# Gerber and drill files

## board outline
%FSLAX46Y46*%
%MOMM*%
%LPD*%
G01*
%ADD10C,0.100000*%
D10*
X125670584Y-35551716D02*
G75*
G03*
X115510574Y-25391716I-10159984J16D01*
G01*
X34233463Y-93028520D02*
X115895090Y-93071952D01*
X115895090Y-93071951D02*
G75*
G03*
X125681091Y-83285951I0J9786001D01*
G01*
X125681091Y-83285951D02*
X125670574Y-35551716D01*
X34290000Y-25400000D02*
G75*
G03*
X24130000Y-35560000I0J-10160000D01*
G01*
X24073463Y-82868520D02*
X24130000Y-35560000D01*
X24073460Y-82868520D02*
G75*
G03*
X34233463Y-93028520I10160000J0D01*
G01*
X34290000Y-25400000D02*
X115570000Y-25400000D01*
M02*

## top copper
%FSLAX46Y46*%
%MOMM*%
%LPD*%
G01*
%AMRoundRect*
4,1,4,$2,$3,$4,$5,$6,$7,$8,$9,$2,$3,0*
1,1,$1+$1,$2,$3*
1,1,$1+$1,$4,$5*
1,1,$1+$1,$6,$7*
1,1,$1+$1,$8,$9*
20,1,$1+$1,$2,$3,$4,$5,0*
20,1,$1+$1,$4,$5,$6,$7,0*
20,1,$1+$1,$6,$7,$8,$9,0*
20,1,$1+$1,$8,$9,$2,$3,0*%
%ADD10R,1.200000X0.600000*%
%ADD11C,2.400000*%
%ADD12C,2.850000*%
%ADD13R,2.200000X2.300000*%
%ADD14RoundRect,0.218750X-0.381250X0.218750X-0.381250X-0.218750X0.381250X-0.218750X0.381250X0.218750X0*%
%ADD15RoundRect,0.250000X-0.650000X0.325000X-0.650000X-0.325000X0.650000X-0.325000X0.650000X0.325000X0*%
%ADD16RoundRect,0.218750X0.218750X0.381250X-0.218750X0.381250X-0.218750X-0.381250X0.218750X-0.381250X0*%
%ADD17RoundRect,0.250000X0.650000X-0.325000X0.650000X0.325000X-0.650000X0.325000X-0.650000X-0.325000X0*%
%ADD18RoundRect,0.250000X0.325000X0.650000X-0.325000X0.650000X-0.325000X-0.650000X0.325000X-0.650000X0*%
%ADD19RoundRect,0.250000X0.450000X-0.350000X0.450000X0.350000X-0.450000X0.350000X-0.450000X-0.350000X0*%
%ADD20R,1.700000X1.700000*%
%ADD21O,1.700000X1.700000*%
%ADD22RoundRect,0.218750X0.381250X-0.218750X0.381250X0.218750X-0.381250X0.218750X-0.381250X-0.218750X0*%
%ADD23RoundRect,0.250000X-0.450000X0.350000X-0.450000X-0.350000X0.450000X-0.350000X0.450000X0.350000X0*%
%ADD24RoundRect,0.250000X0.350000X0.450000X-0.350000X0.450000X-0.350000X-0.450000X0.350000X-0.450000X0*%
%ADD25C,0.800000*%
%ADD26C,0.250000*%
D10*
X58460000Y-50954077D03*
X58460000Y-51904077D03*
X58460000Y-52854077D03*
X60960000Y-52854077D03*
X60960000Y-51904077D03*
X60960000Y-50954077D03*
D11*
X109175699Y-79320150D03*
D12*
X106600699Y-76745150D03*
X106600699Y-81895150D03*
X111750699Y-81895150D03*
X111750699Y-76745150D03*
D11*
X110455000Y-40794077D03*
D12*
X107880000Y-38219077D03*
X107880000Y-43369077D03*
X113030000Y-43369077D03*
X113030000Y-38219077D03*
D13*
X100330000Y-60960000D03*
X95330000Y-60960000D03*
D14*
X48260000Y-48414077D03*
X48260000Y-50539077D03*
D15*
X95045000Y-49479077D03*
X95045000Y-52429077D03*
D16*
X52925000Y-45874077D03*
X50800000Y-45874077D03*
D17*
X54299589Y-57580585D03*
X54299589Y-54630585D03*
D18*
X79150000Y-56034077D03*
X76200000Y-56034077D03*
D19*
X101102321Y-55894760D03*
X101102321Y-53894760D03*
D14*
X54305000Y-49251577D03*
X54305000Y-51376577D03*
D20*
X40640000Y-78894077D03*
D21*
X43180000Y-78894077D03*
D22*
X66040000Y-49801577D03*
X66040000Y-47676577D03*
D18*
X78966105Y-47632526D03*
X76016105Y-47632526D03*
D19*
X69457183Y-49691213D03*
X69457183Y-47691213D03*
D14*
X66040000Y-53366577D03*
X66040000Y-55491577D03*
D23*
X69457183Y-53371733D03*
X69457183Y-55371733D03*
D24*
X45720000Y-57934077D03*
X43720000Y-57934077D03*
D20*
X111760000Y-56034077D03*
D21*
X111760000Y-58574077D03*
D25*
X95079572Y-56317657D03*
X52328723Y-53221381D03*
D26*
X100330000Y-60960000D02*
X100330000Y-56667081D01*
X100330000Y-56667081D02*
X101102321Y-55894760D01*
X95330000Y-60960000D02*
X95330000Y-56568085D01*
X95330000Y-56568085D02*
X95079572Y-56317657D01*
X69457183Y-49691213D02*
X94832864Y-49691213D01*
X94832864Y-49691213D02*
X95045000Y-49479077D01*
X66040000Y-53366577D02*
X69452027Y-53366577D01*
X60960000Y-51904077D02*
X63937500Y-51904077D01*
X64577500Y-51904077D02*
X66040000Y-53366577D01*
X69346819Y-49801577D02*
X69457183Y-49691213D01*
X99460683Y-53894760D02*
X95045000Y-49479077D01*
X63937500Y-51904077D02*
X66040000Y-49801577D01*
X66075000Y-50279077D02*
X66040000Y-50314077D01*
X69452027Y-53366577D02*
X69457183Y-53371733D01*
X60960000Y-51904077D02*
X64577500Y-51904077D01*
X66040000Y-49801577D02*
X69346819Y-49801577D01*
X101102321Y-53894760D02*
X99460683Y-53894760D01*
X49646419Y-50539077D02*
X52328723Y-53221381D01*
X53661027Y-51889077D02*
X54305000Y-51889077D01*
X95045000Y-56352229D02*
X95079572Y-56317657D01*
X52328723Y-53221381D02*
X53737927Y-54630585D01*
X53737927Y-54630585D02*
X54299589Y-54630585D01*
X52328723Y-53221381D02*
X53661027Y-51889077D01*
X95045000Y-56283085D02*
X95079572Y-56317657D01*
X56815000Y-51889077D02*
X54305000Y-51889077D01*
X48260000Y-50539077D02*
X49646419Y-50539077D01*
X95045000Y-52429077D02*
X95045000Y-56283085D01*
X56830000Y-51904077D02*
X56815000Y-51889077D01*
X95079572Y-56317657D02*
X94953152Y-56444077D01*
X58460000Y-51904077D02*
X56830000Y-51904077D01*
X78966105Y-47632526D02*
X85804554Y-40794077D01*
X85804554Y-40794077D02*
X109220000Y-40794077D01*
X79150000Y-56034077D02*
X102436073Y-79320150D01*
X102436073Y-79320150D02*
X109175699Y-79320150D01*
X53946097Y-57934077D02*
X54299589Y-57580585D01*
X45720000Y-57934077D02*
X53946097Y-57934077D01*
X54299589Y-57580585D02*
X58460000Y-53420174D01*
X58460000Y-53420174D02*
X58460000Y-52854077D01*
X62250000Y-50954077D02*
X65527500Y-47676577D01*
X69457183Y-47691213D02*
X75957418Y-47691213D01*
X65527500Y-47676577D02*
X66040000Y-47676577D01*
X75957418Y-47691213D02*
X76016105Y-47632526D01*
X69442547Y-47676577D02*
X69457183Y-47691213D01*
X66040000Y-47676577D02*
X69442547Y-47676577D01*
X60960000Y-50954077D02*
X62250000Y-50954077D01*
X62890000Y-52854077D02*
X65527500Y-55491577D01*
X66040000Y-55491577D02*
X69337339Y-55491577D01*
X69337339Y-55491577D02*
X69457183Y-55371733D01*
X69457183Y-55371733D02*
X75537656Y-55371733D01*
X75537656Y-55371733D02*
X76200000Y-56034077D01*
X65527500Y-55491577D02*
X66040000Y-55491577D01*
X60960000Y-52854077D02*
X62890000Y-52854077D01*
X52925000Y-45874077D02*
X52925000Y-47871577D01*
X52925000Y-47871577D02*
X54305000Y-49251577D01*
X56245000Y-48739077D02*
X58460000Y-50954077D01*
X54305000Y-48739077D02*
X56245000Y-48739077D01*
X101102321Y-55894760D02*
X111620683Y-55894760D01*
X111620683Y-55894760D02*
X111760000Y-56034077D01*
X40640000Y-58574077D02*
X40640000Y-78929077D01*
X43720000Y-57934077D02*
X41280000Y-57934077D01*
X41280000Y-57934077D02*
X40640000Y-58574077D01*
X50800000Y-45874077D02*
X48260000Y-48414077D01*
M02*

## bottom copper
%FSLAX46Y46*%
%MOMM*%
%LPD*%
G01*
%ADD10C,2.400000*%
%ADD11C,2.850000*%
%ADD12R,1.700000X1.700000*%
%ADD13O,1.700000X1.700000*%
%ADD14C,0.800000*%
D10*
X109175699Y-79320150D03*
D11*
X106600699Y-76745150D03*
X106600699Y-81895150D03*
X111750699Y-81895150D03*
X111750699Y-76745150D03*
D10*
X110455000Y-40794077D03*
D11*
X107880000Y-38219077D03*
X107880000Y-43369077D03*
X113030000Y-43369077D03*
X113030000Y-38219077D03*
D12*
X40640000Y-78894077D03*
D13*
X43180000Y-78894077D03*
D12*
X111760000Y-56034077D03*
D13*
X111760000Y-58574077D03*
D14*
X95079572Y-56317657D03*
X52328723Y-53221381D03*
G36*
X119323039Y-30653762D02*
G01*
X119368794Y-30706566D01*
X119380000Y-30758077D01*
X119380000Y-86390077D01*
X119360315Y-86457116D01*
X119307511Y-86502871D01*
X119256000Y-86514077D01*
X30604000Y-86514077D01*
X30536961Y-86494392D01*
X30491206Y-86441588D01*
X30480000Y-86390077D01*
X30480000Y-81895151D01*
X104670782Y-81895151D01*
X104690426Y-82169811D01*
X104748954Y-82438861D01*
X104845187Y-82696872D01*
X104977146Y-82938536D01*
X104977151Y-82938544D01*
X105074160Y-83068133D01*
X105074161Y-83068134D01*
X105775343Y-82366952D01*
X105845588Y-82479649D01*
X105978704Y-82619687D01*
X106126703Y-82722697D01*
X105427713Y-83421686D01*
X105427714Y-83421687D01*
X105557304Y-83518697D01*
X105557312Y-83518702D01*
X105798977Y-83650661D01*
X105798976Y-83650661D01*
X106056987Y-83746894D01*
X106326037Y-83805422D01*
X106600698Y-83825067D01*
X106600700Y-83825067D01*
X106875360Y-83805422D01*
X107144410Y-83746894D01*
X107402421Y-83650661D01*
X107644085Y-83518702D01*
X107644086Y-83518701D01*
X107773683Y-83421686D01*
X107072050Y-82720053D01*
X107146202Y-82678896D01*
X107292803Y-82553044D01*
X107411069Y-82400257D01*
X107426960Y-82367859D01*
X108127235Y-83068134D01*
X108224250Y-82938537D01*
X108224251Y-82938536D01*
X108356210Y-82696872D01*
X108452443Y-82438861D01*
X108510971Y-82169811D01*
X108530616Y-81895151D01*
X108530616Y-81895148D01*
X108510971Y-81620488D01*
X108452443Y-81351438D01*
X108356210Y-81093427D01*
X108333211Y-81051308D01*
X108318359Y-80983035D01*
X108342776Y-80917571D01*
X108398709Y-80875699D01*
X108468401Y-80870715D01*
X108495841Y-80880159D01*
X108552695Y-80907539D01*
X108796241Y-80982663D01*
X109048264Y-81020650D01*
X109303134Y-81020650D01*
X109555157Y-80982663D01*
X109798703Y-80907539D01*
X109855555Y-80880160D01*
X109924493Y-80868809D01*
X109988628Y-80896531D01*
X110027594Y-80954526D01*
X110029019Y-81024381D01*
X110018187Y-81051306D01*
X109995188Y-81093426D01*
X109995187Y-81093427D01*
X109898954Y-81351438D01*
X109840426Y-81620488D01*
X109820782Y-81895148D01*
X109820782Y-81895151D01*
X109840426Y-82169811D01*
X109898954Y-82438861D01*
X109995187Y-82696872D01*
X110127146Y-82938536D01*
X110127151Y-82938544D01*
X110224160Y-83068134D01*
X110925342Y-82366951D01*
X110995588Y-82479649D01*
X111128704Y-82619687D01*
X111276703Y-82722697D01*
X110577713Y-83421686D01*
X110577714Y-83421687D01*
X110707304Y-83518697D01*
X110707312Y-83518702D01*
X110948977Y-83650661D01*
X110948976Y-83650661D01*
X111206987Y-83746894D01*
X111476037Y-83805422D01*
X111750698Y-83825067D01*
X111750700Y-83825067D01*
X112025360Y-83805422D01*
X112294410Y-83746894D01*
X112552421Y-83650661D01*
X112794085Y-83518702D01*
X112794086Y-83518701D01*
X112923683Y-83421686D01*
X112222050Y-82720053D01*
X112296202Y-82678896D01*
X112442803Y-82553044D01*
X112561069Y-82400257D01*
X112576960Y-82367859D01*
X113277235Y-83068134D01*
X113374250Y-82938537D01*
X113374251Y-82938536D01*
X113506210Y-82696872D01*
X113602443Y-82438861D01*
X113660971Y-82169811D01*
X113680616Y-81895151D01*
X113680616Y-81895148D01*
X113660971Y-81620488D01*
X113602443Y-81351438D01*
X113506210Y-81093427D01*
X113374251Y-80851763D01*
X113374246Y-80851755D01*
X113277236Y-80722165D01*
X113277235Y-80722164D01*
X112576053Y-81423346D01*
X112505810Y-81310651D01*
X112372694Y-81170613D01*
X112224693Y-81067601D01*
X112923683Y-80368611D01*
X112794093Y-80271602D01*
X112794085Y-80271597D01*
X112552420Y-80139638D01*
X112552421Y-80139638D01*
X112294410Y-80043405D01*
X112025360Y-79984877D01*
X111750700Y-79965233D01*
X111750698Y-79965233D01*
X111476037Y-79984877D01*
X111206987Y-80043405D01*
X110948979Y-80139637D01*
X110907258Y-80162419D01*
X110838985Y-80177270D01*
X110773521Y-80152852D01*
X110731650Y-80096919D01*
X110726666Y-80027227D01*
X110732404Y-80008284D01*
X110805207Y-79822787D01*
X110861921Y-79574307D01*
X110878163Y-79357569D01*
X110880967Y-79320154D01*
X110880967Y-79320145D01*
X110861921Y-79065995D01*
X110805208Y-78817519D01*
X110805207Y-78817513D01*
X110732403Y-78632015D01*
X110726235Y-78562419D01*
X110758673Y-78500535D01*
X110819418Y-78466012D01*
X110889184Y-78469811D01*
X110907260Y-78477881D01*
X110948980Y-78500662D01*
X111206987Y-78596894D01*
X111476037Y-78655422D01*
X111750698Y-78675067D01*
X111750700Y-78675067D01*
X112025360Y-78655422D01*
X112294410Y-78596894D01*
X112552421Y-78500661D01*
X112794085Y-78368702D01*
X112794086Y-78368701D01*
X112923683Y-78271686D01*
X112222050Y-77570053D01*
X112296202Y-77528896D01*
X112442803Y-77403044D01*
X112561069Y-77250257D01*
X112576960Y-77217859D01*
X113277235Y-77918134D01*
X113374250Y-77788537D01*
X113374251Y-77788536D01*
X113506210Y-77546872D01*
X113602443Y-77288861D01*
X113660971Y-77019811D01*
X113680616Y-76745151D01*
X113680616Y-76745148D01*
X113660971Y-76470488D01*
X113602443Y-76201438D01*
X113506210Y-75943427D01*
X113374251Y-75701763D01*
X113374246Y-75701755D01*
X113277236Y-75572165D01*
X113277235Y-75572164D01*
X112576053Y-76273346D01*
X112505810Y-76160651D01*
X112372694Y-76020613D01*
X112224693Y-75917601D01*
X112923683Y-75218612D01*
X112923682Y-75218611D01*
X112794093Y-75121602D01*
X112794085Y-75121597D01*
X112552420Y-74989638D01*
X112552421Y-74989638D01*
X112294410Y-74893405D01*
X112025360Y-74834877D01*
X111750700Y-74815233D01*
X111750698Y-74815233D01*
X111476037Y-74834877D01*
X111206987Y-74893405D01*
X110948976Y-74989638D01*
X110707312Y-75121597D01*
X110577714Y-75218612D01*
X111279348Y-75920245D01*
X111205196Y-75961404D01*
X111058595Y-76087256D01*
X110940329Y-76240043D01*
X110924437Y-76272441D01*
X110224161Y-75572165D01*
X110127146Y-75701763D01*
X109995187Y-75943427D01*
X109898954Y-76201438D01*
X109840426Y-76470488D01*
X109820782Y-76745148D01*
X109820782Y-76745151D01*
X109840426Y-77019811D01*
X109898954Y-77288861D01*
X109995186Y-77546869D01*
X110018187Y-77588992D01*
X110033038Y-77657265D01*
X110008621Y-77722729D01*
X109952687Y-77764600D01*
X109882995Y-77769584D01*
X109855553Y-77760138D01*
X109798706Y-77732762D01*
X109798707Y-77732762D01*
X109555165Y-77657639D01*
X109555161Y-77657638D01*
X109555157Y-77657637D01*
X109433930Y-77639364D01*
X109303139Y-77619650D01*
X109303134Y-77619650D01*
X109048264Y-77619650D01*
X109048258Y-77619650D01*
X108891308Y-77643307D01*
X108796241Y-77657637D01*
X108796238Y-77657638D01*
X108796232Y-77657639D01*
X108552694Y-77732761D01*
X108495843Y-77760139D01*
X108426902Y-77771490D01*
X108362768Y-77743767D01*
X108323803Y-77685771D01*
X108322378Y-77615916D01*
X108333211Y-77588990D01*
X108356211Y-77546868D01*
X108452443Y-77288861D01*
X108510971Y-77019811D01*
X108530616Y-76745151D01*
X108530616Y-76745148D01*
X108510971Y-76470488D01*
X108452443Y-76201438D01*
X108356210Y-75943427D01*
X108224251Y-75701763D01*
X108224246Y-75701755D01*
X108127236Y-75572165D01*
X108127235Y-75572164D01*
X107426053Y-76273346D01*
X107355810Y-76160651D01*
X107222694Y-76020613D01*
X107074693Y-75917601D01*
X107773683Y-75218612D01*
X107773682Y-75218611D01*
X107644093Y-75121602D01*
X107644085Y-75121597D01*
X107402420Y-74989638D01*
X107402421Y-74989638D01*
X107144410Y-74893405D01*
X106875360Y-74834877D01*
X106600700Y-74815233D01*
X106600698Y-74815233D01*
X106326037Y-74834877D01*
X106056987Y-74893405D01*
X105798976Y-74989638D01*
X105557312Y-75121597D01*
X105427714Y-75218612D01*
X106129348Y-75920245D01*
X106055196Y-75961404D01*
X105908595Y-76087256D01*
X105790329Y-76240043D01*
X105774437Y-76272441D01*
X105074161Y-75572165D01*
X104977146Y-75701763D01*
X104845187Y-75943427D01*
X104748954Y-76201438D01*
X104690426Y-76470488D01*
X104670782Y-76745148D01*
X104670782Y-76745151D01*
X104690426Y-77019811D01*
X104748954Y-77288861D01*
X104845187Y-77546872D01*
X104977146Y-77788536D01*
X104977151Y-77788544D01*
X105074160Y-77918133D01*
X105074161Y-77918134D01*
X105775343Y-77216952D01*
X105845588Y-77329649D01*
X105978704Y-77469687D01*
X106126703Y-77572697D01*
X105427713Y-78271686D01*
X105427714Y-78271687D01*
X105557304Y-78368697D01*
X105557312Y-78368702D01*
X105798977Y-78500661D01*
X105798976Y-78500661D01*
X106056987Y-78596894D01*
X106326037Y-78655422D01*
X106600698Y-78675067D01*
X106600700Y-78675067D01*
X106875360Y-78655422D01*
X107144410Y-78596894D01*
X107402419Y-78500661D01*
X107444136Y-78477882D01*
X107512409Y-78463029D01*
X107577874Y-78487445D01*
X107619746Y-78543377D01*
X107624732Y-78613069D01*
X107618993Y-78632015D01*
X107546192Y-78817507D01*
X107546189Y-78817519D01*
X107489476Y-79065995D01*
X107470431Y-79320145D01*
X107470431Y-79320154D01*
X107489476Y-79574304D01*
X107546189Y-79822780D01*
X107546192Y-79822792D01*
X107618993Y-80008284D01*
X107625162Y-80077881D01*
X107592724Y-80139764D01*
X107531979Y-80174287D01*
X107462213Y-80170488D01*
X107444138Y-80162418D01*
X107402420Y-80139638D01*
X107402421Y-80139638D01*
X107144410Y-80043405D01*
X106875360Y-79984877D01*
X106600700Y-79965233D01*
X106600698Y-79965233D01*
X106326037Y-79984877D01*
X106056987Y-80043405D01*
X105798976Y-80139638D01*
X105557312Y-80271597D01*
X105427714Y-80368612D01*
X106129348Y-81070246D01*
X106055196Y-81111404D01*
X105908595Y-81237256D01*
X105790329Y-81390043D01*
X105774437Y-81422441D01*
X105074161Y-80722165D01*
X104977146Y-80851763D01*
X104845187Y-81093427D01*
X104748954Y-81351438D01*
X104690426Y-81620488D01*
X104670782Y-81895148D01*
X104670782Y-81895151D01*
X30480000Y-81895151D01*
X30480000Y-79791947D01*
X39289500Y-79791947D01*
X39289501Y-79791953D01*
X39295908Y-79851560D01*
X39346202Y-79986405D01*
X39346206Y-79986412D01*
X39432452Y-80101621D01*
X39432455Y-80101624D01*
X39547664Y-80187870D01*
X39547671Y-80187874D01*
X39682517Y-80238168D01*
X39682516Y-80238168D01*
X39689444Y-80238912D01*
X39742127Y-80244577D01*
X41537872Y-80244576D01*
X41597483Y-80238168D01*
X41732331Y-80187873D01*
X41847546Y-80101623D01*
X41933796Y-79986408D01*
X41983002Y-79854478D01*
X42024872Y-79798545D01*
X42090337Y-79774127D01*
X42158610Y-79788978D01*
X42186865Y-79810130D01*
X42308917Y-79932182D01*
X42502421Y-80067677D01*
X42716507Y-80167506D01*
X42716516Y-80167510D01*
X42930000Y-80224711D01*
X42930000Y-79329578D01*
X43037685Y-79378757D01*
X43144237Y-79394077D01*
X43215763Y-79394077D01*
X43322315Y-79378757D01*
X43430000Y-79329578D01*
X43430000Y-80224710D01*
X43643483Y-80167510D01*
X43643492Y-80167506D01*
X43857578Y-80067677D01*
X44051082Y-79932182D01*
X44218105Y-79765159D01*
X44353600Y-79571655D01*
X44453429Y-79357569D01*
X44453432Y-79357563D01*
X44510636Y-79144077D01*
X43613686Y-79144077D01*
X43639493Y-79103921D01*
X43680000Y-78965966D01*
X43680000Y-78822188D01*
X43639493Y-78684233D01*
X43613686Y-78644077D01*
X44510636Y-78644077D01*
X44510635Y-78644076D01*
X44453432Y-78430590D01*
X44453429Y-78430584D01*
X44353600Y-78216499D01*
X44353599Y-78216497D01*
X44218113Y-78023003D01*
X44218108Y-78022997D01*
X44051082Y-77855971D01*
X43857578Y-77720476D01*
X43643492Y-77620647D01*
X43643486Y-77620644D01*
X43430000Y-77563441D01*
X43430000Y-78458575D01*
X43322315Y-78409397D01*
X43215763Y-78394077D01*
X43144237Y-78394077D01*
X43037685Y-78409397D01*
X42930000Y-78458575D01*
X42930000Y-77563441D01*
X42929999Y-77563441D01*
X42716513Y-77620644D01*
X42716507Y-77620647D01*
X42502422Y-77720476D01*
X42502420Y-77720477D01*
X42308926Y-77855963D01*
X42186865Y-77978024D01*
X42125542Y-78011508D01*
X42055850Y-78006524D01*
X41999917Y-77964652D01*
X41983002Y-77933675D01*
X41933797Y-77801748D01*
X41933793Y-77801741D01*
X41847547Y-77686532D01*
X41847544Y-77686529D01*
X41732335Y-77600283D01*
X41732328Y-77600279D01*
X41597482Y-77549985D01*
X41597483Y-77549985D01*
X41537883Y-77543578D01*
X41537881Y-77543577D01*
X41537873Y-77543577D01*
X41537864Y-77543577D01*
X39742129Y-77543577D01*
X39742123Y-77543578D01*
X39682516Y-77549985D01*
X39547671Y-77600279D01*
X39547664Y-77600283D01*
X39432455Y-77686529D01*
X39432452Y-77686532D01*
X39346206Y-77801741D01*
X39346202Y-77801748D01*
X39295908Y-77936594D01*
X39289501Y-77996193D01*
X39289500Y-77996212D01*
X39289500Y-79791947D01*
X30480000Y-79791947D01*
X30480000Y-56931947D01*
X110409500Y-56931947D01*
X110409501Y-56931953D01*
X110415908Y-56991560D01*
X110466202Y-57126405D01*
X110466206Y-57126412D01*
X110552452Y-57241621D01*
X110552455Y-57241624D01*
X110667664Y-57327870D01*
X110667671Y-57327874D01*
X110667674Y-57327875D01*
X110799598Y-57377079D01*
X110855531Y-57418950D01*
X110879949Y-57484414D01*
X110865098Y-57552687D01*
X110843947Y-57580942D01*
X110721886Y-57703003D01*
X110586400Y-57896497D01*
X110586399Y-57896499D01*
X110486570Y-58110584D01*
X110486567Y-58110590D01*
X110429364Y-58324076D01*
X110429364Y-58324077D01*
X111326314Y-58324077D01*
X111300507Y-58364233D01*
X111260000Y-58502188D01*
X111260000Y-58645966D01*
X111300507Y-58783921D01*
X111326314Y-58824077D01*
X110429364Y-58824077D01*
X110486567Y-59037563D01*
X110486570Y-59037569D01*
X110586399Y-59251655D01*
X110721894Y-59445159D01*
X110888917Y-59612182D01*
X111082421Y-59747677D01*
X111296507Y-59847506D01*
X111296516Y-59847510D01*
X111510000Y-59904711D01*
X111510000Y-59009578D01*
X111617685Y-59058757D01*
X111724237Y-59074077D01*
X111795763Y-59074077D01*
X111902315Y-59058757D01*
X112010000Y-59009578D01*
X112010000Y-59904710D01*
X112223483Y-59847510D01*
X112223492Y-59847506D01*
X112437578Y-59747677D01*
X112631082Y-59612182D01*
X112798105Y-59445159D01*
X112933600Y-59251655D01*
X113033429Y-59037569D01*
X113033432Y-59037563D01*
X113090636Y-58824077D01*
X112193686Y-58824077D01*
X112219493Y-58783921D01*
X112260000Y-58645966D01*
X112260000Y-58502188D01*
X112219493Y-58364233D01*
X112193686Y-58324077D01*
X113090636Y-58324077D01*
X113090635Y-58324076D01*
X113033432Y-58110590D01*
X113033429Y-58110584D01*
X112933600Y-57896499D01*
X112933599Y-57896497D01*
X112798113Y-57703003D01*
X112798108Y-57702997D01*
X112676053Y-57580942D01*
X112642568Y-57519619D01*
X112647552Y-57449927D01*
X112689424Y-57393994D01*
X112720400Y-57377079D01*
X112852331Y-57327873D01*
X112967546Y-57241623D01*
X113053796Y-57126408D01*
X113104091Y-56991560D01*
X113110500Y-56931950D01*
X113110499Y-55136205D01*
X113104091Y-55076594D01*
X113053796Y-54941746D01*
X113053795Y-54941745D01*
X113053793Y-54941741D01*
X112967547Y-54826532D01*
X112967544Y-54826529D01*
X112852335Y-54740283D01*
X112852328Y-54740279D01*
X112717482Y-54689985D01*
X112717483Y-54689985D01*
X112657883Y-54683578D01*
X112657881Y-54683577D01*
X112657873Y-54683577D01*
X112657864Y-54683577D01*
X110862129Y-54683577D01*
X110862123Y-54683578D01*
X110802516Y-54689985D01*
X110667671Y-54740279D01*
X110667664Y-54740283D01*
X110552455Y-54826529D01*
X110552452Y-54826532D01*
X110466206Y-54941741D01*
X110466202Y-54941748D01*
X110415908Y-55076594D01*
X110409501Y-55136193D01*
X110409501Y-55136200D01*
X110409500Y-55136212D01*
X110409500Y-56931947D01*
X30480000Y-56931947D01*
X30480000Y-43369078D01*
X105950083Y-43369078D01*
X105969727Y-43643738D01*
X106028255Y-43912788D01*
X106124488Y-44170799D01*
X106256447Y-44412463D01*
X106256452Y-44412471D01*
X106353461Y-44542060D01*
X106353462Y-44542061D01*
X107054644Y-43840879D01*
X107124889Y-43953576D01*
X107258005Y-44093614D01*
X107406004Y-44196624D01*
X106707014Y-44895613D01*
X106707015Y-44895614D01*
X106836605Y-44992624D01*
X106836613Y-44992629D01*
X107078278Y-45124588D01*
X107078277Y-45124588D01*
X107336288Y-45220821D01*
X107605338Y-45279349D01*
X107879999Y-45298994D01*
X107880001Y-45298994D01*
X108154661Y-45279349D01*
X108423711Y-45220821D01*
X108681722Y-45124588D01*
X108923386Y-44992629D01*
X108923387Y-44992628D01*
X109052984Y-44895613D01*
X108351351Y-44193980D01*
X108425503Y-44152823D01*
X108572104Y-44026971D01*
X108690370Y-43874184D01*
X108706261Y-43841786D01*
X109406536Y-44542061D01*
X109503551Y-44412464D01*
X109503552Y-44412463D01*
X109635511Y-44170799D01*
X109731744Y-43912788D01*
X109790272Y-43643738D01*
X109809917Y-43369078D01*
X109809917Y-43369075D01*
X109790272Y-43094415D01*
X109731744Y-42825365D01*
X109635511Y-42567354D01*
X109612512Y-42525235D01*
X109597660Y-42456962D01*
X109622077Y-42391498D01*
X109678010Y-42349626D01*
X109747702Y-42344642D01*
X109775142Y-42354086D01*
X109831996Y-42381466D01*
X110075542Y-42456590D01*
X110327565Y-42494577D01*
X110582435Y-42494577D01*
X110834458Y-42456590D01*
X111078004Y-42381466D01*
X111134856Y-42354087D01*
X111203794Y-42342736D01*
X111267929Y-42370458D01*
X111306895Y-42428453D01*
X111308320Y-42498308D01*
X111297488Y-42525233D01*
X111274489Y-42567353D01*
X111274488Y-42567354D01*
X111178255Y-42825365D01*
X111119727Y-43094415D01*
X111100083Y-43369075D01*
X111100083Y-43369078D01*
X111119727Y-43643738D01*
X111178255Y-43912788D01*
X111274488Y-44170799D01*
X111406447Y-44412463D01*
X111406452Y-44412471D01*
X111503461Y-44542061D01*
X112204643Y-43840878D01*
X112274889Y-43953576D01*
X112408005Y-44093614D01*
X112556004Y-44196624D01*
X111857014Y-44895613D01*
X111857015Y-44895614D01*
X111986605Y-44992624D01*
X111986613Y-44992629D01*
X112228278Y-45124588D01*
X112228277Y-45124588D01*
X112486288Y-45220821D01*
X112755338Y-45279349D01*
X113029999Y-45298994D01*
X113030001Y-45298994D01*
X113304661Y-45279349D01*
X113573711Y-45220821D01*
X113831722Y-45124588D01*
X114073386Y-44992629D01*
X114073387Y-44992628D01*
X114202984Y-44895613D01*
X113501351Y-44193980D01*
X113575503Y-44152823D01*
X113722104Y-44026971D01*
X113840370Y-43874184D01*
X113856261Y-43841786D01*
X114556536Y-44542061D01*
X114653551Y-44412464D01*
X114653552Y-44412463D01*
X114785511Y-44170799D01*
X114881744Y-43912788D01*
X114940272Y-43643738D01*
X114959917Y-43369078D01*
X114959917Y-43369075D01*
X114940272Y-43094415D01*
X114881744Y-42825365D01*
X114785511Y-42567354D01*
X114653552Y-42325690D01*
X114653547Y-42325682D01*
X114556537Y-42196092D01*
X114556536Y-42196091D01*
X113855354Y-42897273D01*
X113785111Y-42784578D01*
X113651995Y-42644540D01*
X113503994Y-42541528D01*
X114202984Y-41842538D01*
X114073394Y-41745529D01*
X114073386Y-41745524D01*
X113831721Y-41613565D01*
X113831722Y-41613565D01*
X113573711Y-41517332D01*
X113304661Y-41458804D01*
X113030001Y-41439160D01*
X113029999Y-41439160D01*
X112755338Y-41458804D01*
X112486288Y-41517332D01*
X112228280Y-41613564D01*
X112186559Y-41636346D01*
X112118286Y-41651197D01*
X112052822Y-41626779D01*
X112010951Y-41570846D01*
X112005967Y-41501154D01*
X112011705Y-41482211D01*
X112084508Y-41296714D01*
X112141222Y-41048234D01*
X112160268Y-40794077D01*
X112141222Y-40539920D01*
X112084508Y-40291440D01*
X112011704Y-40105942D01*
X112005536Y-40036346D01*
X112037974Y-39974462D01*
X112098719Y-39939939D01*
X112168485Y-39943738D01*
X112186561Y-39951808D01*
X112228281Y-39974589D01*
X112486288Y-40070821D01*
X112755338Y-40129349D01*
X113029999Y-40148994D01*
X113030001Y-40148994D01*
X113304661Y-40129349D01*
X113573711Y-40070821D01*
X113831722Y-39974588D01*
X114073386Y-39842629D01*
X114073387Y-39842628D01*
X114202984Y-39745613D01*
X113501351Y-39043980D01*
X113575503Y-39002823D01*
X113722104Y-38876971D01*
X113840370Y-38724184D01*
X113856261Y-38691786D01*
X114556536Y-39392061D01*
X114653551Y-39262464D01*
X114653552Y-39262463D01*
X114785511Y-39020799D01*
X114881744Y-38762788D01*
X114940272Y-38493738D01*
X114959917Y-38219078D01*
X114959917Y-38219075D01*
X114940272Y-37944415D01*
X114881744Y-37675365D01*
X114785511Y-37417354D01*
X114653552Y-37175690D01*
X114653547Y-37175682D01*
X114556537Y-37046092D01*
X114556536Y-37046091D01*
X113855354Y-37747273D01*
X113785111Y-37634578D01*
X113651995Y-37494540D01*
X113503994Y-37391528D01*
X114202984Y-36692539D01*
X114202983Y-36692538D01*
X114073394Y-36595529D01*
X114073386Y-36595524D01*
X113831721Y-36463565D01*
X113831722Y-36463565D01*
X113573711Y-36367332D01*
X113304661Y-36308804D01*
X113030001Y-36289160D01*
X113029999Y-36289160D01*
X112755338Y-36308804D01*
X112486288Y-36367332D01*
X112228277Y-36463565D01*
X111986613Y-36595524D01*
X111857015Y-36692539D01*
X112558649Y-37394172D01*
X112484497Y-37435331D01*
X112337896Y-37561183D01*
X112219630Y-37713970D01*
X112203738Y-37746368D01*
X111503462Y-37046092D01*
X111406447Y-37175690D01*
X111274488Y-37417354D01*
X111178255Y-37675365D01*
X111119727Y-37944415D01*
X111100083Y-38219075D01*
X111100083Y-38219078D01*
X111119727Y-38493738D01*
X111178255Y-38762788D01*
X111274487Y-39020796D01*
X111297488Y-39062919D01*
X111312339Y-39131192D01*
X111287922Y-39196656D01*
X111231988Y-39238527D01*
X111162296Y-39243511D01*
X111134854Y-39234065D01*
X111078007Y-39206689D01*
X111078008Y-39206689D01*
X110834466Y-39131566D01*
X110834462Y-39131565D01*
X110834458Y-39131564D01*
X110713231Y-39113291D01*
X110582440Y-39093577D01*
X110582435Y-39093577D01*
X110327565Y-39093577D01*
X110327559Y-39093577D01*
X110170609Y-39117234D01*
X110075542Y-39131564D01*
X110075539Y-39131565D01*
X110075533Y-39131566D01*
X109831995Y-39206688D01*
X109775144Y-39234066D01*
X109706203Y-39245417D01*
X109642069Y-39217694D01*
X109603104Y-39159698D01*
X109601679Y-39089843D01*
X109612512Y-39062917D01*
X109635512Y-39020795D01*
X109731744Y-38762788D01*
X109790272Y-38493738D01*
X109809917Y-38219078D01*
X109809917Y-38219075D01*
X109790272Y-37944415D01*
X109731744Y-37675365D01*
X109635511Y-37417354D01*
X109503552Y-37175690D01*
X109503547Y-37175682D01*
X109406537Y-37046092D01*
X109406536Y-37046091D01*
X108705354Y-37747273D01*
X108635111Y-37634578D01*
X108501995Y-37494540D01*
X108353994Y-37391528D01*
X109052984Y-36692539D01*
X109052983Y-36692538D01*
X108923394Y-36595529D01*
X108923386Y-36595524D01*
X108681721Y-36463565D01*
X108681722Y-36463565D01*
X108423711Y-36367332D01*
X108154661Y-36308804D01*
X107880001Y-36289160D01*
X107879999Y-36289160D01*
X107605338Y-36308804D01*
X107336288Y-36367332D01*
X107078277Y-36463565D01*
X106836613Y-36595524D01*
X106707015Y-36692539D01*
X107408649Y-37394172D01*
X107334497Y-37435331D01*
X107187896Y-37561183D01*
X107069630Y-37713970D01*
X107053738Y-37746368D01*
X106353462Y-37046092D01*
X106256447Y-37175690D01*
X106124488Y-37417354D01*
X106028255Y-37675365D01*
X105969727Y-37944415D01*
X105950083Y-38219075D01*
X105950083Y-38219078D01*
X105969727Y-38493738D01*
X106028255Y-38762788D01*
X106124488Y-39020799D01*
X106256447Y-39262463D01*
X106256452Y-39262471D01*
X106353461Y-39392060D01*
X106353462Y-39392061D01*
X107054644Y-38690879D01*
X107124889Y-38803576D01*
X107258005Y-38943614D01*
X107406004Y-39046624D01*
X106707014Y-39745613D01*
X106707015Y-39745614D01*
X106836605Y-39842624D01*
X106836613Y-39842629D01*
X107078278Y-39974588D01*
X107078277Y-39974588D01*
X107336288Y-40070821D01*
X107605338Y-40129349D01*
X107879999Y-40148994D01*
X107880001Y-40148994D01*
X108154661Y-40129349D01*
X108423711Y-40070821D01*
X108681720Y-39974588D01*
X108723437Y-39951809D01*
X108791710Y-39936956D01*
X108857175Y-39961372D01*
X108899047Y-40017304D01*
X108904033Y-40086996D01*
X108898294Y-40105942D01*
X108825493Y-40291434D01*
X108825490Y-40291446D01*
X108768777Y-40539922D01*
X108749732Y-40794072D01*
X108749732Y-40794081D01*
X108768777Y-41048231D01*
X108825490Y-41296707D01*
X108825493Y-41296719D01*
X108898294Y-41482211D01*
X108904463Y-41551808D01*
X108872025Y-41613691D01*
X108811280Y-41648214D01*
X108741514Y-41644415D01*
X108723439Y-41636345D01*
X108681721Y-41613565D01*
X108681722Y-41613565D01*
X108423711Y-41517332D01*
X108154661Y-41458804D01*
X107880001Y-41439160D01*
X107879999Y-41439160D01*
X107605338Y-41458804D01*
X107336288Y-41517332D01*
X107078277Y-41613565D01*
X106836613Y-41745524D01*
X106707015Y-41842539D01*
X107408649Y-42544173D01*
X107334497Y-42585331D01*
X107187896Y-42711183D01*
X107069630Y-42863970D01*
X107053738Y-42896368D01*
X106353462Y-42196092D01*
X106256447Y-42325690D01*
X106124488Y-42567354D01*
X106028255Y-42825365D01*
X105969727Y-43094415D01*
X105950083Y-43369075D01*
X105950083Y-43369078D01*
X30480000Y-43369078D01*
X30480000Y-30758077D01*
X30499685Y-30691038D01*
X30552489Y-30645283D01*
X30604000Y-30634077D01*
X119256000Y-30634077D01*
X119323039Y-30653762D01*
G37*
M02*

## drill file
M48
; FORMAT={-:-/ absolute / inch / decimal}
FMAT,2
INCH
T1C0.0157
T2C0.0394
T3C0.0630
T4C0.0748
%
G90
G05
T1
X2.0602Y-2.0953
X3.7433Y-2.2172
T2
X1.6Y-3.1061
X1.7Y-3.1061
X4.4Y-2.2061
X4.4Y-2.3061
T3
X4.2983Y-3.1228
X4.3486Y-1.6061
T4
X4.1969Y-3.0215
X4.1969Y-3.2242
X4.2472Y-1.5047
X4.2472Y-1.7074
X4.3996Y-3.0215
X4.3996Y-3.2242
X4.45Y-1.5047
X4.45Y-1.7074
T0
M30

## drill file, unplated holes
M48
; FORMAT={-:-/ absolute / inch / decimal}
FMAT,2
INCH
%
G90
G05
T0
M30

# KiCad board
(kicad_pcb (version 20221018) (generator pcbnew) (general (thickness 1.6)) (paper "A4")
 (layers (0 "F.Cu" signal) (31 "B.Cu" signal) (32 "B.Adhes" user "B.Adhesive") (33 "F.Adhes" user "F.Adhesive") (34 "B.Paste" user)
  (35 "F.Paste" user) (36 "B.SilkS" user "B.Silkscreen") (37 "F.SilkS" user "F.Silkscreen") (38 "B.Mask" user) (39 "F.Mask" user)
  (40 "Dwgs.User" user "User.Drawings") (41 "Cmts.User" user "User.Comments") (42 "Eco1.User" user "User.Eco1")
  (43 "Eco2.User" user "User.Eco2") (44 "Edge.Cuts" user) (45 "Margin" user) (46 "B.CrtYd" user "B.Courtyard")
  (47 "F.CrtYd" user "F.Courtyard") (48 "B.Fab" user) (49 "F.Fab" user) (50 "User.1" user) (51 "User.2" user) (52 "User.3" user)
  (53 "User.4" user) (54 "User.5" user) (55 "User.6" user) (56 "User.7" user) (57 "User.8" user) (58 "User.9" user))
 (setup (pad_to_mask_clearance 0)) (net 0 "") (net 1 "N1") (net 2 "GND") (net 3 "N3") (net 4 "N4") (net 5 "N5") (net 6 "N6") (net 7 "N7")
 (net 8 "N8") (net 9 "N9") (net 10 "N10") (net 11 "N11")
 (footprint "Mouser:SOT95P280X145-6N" (layer "F.Cu") (at 59.71 51.904077)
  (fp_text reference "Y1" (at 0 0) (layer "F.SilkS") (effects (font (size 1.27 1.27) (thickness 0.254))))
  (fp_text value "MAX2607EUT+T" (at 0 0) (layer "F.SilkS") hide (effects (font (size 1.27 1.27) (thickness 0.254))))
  (pad "1" smd rect (at -1.25 -0.95 90) (size 0.6 1.2) (layers "F.Cu" "F.Paste" "F.Mask") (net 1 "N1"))
  (pad "2" smd rect (at -1.25 0 90) (size 0.6 1.2) (layers "F.Cu" "F.Paste" "F.Mask") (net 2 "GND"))
  (pad "3" smd rect (at -1.25 0.95 90) (size 0.6 1.2) (layers "F.Cu" "F.Paste" "F.Mask") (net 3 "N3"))
  (pad "4" smd rect (at 1.25 0.95 90) (size 0.6 1.2) (layers "F.Cu" "F.Paste" "F.Mask") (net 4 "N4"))
  (pad "5" smd rect (at 1.25 0 90) (size 0.6 1.2) (layers "F.Cu" "F.Paste" "F.Mask") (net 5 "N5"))
  (pad "6" smd rect (at 1.25 -0.95 90) (size 0.6 1.2) (layers "F.Cu" "F.Paste" "F.Mask") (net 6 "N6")))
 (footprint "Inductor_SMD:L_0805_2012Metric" (layer "F.Cu") (at 48.26 49.476577 -90)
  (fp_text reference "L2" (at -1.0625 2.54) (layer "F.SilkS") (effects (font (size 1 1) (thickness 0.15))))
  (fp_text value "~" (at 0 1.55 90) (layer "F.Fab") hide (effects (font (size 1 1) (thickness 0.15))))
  (pad "1" smd roundrect (at -1.0625 0 270) (size 0.875 1.2) (layers "F.Cu" "F.Paste" "F.Mask") (roundrect_rratio 0.25) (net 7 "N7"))
  (pad "2" smd roundrect (at 1.0625 0 270) (size 0.875 1.2) (layers "F.Cu" "F.Paste" "F.Mask") (roundrect_rratio 0.25) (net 2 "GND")))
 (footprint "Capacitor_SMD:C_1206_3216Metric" (layer "F.Cu") (at 95.045 50.954077 -90)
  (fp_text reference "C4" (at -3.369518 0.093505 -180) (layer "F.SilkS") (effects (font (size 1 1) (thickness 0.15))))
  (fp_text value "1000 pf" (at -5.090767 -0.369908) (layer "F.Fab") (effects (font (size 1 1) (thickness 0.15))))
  (pad "1" smd roundrect (at -1.475 0 270) (size 1.15 1.8) (layers "F.Cu" "F.Paste" "F.Mask") (roundrect_rratio 0.2173913043) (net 5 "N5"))
  (pad "2" smd roundrect (at 1.475 0 270) (size 1.15 1.8) (layers "F.Cu" "F.Paste" "F.Mask") (roundrect_rratio 0.2173913043) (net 2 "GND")))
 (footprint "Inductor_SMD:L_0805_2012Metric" (layer "F.Cu") (at 51.8625 45.874077 180)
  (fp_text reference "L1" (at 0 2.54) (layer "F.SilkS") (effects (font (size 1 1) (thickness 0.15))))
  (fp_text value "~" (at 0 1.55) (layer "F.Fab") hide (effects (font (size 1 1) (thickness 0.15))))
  (pad "1" smd roundrect (at -1.0625 0 180) (size 0.875 1.2) (layers "F.Cu" "F.Paste" "F.Mask") (roundrect_rratio 0.25) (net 1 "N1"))
  (pad "2" smd roundrect (at 1.0625 0 180) (size 0.875 1.2) (layers "F.Cu" "F.Paste" "F.Mask") (roundrect_rratio 0.25) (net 7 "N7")))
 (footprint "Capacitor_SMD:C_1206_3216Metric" (layer "F.Cu") (at 54.299589 56.105585 90)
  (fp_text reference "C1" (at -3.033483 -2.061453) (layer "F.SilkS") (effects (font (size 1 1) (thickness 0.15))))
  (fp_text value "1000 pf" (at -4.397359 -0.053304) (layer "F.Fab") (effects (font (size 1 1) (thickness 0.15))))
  (pad "1" smd roundrect (at -1.475 0 90) (size 1.15 1.8) (layers "F.Cu" "F.Paste" "F.Mask") (roundrect_rratio 0.2173913043) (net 3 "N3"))
  (pad "2" smd roundrect (at 1.475 0 90) (size 1.15 1.8) (layers "F.Cu" "F.Paste" "F.Mask") (roundrect_rratio 0.2173913043) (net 2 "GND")))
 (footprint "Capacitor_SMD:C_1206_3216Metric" (layer "F.Cu") (at 77.675 56.034077 180)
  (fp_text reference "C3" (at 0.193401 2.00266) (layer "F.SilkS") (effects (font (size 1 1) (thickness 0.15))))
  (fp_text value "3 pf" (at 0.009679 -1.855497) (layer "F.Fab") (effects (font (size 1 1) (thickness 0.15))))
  (pad "1" smd roundrect (at -1.475 0 180) (size 1.15 1.8) (layers "F.Cu" "F.Paste" "F.Mask") (roundrect_rratio 0.2173913043) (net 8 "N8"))
  (pad "2" smd roundrect (at 1.475 0 180) (size 1.15 1.8) (layers "F.Cu" "F.Paste" "F.Mask") (roundrect_rratio 0.2173913043) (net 4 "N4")))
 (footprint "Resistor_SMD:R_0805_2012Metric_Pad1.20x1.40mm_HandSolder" (layer "F.Cu") (at 101.102321 54.89476 90)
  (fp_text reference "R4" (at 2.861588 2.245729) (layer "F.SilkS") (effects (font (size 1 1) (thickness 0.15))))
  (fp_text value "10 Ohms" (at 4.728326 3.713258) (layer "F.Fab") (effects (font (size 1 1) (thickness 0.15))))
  (pad "1" smd roundrect (at -1 0 90) (size 1.2 1.4) (layers "F.Cu" "F.Paste" "F.Mask") (roundrect_rratio 0.2083333333) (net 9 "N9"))
  (pad "2" smd roundrect (at 1 0 90) (size 1.2 1.4) (layers "F.Cu" "F.Paste" "F.Mask") (roundrect_rratio 0.2083333333) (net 5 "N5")))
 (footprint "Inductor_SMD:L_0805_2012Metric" (layer "F.Cu") (at 54.305 50.314077 -90)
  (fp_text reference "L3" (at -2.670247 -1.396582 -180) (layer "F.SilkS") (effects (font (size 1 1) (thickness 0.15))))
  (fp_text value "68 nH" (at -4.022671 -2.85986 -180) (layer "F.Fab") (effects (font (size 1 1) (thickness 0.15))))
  (pad "1" smd roundrect (at -1.0625 0 270) (size 0.875 1.2) (layers "F.Cu" "F.Paste" "F.Mask") (roundrect_rratio 0.25) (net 1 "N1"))
  (pad "2" smd roundrect (at 1.0625 0 270) (size 0.875 1.2) (layers "F.Cu" "F.Paste" "F.Mask") (roundrect_rratio 0.25) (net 2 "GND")))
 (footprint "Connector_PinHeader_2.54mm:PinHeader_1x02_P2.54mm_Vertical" (layer "F.Cu") (at 40.64 78.894077 90)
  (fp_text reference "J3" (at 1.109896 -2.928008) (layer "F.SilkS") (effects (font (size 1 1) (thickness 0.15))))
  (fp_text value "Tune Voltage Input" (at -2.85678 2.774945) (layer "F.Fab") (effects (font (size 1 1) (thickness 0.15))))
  (pad "1" thru_hole rect (at 0 0 90) (size 1.7 1.7) (drill 1) (layers "*.Cu" "*.Mask") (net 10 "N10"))
  (pad "2" thru_hole oval (at 0 2.54 90) (size 1.7 1.7) (drill 1) (layers "*.Cu" "*.Mask") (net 2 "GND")))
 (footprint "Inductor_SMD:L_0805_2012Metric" (layer "F.Cu") (at 66.04 48.739077 90)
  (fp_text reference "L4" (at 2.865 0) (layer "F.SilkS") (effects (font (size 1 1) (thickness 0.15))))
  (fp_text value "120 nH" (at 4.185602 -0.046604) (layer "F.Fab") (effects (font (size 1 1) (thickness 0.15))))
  (pad "1" smd roundrect (at -1.0625 0 90) (size 0.875 1.2) (layers "F.Cu" "F.Paste" "F.Mask") (roundrect_rratio 0.25) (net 5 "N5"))
  (pad "2" smd roundrect (at 1.0625 0 90) (size 0.875 1.2) (layers "F.Cu" "F.Paste" "F.Mask") (roundrect_rratio 0.25) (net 6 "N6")))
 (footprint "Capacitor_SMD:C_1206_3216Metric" (layer "F.Cu") (at 77.491105 47.632526 180)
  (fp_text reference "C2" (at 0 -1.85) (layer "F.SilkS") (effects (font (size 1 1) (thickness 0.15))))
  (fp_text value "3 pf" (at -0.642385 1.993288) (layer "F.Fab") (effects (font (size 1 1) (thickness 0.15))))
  (pad "1" smd roundrect (at -1.475 0 180) (size 1.15 1.8) (layers "F.Cu" "F.Paste" "F.Mask") (roundrect_rratio 0.2173913043) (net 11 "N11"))
  (pad "2" smd roundrect (at 1.475 0 180) (size 1.15 1.8) (layers "F.Cu" "F.Paste" "F.Mask") (roundrect_rratio 0.2173913043) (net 6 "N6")))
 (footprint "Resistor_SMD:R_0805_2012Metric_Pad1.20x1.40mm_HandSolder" (layer "F.Cu") (at 69.457183 48.691213 90)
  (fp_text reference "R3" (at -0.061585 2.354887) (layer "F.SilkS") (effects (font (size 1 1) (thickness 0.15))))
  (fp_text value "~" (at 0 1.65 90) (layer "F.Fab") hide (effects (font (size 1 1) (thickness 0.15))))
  (pad "1" smd roundrect (at -1 0 90) (size 1.2 1.4) (layers "F.Cu" "F.Paste" "F.Mask") (roundrect_rratio 0.2083333333) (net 5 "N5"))
  (pad "2" smd roundrect (at 1 0 90) (size 1.2 1.4) (layers "F.Cu" "F.Paste" "F.Mask") (roundrect_rratio 0.2083333333) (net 6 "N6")))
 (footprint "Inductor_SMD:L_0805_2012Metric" (layer "F.Cu") (at 66.04 54.429077 -90)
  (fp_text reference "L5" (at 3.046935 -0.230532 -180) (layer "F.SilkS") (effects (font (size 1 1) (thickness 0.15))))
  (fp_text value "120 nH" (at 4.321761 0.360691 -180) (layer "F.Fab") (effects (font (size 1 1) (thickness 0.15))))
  (pad "1" smd roundrect (at -1.0625 0 270) (size 0.875 1.2) (layers "F.Cu" "F.Paste" "F.Mask") (roundrect_rratio 0.25) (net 5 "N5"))
  (pad "2" smd roundrect (at 1.0625 0 270) (size 0.875 1.2) (layers "F.Cu" "F.Paste" "F.Mask") (roundrect_rratio 0.25) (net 4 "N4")))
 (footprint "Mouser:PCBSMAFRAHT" (layer "F.Cu") (at 110.455 40.794077)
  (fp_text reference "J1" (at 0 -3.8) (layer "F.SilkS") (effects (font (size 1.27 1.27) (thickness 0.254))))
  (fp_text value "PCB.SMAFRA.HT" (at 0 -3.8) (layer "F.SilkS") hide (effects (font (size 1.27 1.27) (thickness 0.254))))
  (pad "1" thru_hole circle (at 0 0) (size 2.4 2.4) (drill 1.6) (layers "*.Cu" "*.Mask") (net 11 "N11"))
  (pad "2" thru_hole circle (at -2.575 -2.575) (size 2.85 2.85) (drill 1.9) (layers "*.Cu" "*.Mask") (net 2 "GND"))
  (pad "3" thru_hole circle (at -2.575 2.575) (size 2.85 2.85) (drill 1.9) (layers "*.Cu" "*.Mask") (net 2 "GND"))
  (pad "4" thru_hole circle (at 2.575 2.575) (size 2.85 2.85) (drill 1.9) (layers "*.Cu" "*.Mask") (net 2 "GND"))
  (pad "5" thru_hole circle (at 2.575 -2.575) (size 2.85 2.85) (drill 1.9) (layers "*.Cu" "*.Mask") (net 2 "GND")))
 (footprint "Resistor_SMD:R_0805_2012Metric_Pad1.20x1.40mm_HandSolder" (layer "F.Cu") (at 69.457183 54.371733 -90)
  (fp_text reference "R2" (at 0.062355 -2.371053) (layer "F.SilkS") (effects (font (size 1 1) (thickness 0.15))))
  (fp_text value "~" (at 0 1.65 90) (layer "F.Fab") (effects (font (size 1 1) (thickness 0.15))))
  (pad "1" smd roundrect (at -1 0 270) (size 1.2 1.4) (layers "F.Cu" "F.Paste" "F.Mask") (roundrect_rratio 0.2083333333) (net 5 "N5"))
  (pad "2" smd roundrect (at 1 0 270) (size 1.2 1.4) (layers "F.Cu" "F.Paste" "F.Mask") (roundrect_rratio 0.2083333333) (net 4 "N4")))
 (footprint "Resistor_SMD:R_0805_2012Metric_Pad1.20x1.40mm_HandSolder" (layer "F.Cu") (at 44.72 57.934077 180)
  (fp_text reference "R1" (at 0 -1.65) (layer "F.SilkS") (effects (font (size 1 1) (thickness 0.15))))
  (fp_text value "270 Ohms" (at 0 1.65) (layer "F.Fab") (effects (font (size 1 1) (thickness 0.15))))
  (pad "1" smd roundrect (at -1 0 180) (size 1.2 1.4) (layers "F.Cu" "F.Paste" "F.Mask") (roundrect_rratio 0.2083333333) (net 3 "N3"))
  (pad "2" smd roundrect (at 1 0 180) (size 1.2 1.4) (layers "F.Cu" "F.Paste" "F.Mask") (roundrect_rratio 0.2083333333) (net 10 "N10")))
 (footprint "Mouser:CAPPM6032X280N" (layer "F.Cu") (at 97.83 60.96 180)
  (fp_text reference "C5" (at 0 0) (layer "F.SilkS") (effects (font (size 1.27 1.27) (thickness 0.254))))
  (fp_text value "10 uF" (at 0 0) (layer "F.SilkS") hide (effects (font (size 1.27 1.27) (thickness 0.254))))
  (pad "1" smd rect (at -2.5 0 180) (size 2.2 2.3) (layers "F.Cu" "F.Paste" "F.Mask") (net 9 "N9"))
  (pad "2" smd rect (at 2.5 0 180) (size 2.2 2.3) (layers "F.Cu" "F.Paste" "F.Mask") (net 2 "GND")))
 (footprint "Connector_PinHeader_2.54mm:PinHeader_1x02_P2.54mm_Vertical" (layer "F.Cu") (at 111.76 56.034077)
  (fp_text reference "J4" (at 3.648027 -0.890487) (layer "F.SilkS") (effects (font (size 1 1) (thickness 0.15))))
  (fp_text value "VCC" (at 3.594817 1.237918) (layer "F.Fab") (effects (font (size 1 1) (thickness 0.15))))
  (pad "1" thru_hole rect (at 0 0) (size 1.7 1.7) (drill 1) (layers "*.Cu" "*.Mask") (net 9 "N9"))
  (pad "2" thru_hole oval (at 0 2.54) (size 1.7 1.7) (drill 1) (layers "*.Cu" "*.Mask") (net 2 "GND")))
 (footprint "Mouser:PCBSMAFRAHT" (layer "F.Cu") (at 109.175699 79.32015)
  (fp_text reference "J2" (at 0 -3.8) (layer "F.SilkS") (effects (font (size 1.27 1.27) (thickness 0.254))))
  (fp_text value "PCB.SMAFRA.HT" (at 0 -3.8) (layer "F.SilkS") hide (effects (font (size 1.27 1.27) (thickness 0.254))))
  (pad "1" thru_hole circle (at 0 0) (size 2.4 2.4) (drill 1.6) (layers "*.Cu" "*.Mask") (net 8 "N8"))
  (pad "2" thru_hole circle (at -2.575 -2.575) (size 2.85 2.85) (drill 1.9) (layers "*.Cu" "*.Mask") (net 2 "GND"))
  (pad "3" thru_hole circle (at -2.575 2.575) (size 2.85 2.85) (drill 1.9) (layers "*.Cu" "*.Mask") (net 2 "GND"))
  (pad "4" thru_hole circle (at 2.575 2.575) (size 2.85 2.85) (drill 1.9) (layers "*.Cu" "*.Mask") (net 2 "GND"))
  (pad "5" thru_hole circle (at 2.575 -2.575) (size 2.85 2.85) (drill 1.9) (layers "*.Cu" "*.Mask") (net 2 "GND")))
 (gr_arc (start 115.510574 25.391716) (mid 122.694779 28.367511) (end 125.670574 35.551716) (stroke (width 0.1) (type default))
  (layer "Edge.Cuts"))
 (gr_line (start 34.233463 93.02852) (end 115.89509 93.071952) (stroke (width 0.1) (type default)) (layer "Edge.Cuts"))
 (gr_arc (start 125.681091 83.285951) (mid 122.814838 90.205699) (end 115.89509 93.071952) (stroke (width 0.1) (type default))
  (layer "Edge.Cuts"))
 (gr_line (start 125.681091 83.285951) (end 125.670574 35.551716) (stroke (width 0.1) (type default)) (layer "Edge.Cuts"))
 (gr_arc (start 24.13 35.56) (mid 27.105795 28.375795) (end 34.29 25.4) (stroke (width 0.1) (type default)) (layer "Edge.Cuts"))
 (gr_line (start 24.073463 82.86852) (end 24.13 35.56) (stroke (width 0.1) (type default)) (layer "Edge.Cuts"))
 (gr_arc (start 34.233463 93.02852) (mid 27.049258 90.052725) (end 24.073463 82.86852) (stroke (width 0.1) (type default))
  (layer "Edge.Cuts"))
 (gr_line (start 34.29 25.4) (end 115.57 25.4) (stroke (width 0.1) (type default)) (layer "Edge.Cuts"))
 (segment (start 69.457183 49.691213) (end 94.832864 49.691213) (width 0.25) (layer "F.Cu") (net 5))
 (segment (start 94.832864 49.691213) (end 95.045 49.479077) (width 0.25) (layer "F.Cu") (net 5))
 (segment (start 66.04 53.366577) (end 69.452027 53.366577) (width 0.25) (layer "F.Cu") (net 5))
 (segment (start 60.96 51.904077) (end 63.9375 51.904077) (width 0.25) (layer "F.Cu") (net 5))
 (segment (start 64.5775 51.904077) (end 66.04 53.366577) (width 0.25) (layer "F.Cu") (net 5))
 (segment (start 69.346819 49.801577) (end 69.457183 49.691213) (width 0.25) (layer "F.Cu") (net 5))
 (segment (start 99.460683 53.89476) (end 95.045 49.479077) (width 0.25) (layer "F.Cu") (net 5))
 (segment (start 63.9375 51.904077) (end 66.04 49.801577) (width 0.25) (layer "F.Cu") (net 5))
 (segment (start 66.075 50.279077) (end 66.04 50.314077) (width 0.25) (layer "F.Cu") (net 5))
 (segment (start 69.452027 53.366577) (end 69.457183 53.371733) (width 0.25) (layer "F.Cu") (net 5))
 (segment (start 60.96 51.904077) (end 64.5775 51.904077) (width 0.25) (layer "F.Cu") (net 5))
 (segment (start 66.04 49.801577) (end 69.346819 49.801577) (width 0.25) (layer "F.Cu") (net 5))
 (segment (start 101.102321 53.89476) (end 99.460683 53.89476) (width 0.25) (layer "F.Cu") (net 5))
 (segment (start 49.646419 50.539077) (end 52.328723 53.221381) (width 0.25) (layer "F.Cu") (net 2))
 (segment (start 95.33 60.96) (end 95.33 56.568085) (width 0.25) (layer "F.Cu") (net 2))
 (segment (start 53.661027 51.889077) (end 54.305 51.889077) (width 0.25) (layer "F.Cu") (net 2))
 (segment (start 95.33 56.568085) (end 95.079572 56.317657) (width 0.25) (layer "F.Cu") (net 2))
 (segment (start 95.045 56.352229) (end 95.079572 56.317657) (width 0.25) (layer "F.Cu") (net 2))
 (segment (start 52.328723 53.221381) (end 53.737927 54.630585) (width 0.25) (layer "F.Cu") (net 2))
 (segment (start 53.737927 54.630585) (end 54.299589 54.630585) (width 0.25) (layer "F.Cu") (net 2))
 (segment (start 52.328723 53.221381) (end 53.661027 51.889077) (width 0.25) (layer "F.Cu") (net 2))
 (segment (start 95.045 56.283085) (end 95.079572 56.317657) (width 0.25) (layer "F.Cu") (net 2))
 (segment (start 56.815 51.889077) (end 54.305 51.889077) (width 0.25) (layer "F.Cu") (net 2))
 (segment (start 48.26 50.539077) (end 49.646419 50.539077) (width 0.25) (layer "F.Cu") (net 2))
 (segment (start 95.045 52.429077) (end 95.045 56.283085) (width 0.25) (layer "F.Cu") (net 2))
 (segment (start 56.83 51.904077) (end 56.815 51.889077) (width 0.25) (layer "F.Cu") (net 2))
 (segment (start 95.079572 56.317657) (end 94.953152 56.444077) (width 0.25) (layer "F.Cu") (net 2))
 (segment (start 58.46 51.904077) (end 56.83 51.904077) (width 0.25) (layer "F.Cu") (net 2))
 (via (at 95.079572 56.317657) (size 0.8) (drill 0.4) (layers "F.Cu" "B.Cu") (free) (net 2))
 (via (at 52.328723 53.221381) (size 0.8) (drill 0.4) (layers "F.Cu" "B.Cu") (free) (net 2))
 (segment (start 78.966105 47.632526) (end 85.804554 40.794077) (width 0.25) (layer "F.Cu") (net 11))
 (segment (start 85.804554 40.794077) (end 109.22 40.794077) (width 0.25) (layer "F.Cu") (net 11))
 (segment (start 79.15 56.034077) (end 102.436073 79.32015) (width 0.25) (layer "F.Cu") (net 8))
 (segment (start 102.436073 79.32015) (end 109.175699 79.32015) (width 0.25) (layer "F.Cu") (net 8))
 (segment (start 53.946097 57.934077) (end 54.299589 57.580585) (width 0.25) (layer "F.Cu") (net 3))
 (segment (start 45.72 57.934077) (end 53.946097 57.934077) (width 0.25) (layer "F.Cu") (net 3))
 (segment (start 54.299589 57.580585) (end 58.46 53.420174) (width 0.25) (layer "F.Cu") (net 3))
 (segment (start 58.46 53.420174) (end 58.46 52.854077) (width 0.25) (layer "F.Cu") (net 3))
 (segment (start 62.25 50.954077) (end 65.5275 47.676577) (width 0.25) (layer "F.Cu") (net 6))
 (segment (start 69.457183 47.691213) (end 75.957418 47.691213) (width 0.25) (layer "F.Cu") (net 6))
 (segment (start 65.5275 47.676577) (end 66.04 47.676577) (width 0.25) (layer "F.Cu") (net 6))
 (segment (start 75.957418 47.691213) (end 76.016105 47.632526) (width 0.25) (layer "F.Cu") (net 6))
 (segment (start 69.442547 47.676577) (end 69.457183 47.691213) (width 0.25) (layer "F.Cu") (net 6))
 (segment (start 66.04 47.676577) (end 69.442547 47.676577) (width 0.25) (layer "F.Cu") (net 6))
 (segment (start 60.96 50.954077) (end 62.25 50.954077) (width 0.25) (layer "F.Cu") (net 6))
 (segment (start 62.89 52.854077) (end 65.5275 55.491577) (width 0.25) (layer "F.Cu") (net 4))
 (segment (start 66.04 55.491577) (end 69.337339 55.491577) (width 0.25) (layer "F.Cu") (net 4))
 (segment (start 69.337339 55.491577) (end 69.457183 55.371733) (width 0.25) (layer "F.Cu") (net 4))
 (segment (start 69.457183 55.371733) (end 75.537656 55.371733) (width 0.25) (layer "F.Cu") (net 4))
 (segment (start 75.537656 55.371733) (end 76.2 56.034077) (width 0.25) (layer "F.Cu") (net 4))
 (segment (start 65.5275 55.491577) (end 66.04 55.491577) (width 0.25) (layer "F.Cu") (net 4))
 (segment (start 60.96 52.854077) (end 62.89 52.854077) (width 0.25) (layer "F.Cu") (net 4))
 (segment (start 52.925 45.874077) (end 52.925 47.871577) (width 0.25) (layer "F.Cu") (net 1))
 (segment (start 52.925 47.871577) (end 54.305 49.251577) (width 0.25) (layer "F.Cu") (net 1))
 (segment (start 56.245 48.739077) (end 58.46 50.954077) (width 0.25) (layer "F.Cu") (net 1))
 (segment (start 54.305 48.739077) (end 56.245 48.739077) (width 0.25) (layer "F.Cu") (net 1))
 (segment (start 40.64 58.574077) (end 40.64 78.929077) (width 0.25) (layer "F.Cu") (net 10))
 (segment (start 43.72 57.934077) (end 41.28 57.934077) (width 0.25) (layer "F.Cu") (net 10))
 (segment (start 41.28 57.934077) (end 40.64 58.574077) (width 0.25) (layer "F.Cu") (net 10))
 (segment (start 50.8 45.874077) (end 48.26 48.414077) (width 0.25) (layer "F.Cu") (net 7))
 (segment (start 100.33 60.96) (end 100.33 56.667081) (width 0.25) (layer "F.Cu") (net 9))
 (segment (start 101.102321 55.89476) (end 111.620683 55.89476) (width 0.25) (layer "F.Cu") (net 9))
 (segment (start 111.620683 55.89476) (end 111.76 56.034077) (width 0.25) (layer "F.Cu") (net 9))
 (segment (start 100.33 56.667081) (end 101.102321 55.89476) (width 0.25) (layer "F.Cu") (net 9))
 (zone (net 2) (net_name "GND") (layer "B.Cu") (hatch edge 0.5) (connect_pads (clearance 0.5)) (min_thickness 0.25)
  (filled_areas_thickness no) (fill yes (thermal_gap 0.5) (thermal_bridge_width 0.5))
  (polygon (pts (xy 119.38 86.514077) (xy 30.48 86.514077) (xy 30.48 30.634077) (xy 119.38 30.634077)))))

